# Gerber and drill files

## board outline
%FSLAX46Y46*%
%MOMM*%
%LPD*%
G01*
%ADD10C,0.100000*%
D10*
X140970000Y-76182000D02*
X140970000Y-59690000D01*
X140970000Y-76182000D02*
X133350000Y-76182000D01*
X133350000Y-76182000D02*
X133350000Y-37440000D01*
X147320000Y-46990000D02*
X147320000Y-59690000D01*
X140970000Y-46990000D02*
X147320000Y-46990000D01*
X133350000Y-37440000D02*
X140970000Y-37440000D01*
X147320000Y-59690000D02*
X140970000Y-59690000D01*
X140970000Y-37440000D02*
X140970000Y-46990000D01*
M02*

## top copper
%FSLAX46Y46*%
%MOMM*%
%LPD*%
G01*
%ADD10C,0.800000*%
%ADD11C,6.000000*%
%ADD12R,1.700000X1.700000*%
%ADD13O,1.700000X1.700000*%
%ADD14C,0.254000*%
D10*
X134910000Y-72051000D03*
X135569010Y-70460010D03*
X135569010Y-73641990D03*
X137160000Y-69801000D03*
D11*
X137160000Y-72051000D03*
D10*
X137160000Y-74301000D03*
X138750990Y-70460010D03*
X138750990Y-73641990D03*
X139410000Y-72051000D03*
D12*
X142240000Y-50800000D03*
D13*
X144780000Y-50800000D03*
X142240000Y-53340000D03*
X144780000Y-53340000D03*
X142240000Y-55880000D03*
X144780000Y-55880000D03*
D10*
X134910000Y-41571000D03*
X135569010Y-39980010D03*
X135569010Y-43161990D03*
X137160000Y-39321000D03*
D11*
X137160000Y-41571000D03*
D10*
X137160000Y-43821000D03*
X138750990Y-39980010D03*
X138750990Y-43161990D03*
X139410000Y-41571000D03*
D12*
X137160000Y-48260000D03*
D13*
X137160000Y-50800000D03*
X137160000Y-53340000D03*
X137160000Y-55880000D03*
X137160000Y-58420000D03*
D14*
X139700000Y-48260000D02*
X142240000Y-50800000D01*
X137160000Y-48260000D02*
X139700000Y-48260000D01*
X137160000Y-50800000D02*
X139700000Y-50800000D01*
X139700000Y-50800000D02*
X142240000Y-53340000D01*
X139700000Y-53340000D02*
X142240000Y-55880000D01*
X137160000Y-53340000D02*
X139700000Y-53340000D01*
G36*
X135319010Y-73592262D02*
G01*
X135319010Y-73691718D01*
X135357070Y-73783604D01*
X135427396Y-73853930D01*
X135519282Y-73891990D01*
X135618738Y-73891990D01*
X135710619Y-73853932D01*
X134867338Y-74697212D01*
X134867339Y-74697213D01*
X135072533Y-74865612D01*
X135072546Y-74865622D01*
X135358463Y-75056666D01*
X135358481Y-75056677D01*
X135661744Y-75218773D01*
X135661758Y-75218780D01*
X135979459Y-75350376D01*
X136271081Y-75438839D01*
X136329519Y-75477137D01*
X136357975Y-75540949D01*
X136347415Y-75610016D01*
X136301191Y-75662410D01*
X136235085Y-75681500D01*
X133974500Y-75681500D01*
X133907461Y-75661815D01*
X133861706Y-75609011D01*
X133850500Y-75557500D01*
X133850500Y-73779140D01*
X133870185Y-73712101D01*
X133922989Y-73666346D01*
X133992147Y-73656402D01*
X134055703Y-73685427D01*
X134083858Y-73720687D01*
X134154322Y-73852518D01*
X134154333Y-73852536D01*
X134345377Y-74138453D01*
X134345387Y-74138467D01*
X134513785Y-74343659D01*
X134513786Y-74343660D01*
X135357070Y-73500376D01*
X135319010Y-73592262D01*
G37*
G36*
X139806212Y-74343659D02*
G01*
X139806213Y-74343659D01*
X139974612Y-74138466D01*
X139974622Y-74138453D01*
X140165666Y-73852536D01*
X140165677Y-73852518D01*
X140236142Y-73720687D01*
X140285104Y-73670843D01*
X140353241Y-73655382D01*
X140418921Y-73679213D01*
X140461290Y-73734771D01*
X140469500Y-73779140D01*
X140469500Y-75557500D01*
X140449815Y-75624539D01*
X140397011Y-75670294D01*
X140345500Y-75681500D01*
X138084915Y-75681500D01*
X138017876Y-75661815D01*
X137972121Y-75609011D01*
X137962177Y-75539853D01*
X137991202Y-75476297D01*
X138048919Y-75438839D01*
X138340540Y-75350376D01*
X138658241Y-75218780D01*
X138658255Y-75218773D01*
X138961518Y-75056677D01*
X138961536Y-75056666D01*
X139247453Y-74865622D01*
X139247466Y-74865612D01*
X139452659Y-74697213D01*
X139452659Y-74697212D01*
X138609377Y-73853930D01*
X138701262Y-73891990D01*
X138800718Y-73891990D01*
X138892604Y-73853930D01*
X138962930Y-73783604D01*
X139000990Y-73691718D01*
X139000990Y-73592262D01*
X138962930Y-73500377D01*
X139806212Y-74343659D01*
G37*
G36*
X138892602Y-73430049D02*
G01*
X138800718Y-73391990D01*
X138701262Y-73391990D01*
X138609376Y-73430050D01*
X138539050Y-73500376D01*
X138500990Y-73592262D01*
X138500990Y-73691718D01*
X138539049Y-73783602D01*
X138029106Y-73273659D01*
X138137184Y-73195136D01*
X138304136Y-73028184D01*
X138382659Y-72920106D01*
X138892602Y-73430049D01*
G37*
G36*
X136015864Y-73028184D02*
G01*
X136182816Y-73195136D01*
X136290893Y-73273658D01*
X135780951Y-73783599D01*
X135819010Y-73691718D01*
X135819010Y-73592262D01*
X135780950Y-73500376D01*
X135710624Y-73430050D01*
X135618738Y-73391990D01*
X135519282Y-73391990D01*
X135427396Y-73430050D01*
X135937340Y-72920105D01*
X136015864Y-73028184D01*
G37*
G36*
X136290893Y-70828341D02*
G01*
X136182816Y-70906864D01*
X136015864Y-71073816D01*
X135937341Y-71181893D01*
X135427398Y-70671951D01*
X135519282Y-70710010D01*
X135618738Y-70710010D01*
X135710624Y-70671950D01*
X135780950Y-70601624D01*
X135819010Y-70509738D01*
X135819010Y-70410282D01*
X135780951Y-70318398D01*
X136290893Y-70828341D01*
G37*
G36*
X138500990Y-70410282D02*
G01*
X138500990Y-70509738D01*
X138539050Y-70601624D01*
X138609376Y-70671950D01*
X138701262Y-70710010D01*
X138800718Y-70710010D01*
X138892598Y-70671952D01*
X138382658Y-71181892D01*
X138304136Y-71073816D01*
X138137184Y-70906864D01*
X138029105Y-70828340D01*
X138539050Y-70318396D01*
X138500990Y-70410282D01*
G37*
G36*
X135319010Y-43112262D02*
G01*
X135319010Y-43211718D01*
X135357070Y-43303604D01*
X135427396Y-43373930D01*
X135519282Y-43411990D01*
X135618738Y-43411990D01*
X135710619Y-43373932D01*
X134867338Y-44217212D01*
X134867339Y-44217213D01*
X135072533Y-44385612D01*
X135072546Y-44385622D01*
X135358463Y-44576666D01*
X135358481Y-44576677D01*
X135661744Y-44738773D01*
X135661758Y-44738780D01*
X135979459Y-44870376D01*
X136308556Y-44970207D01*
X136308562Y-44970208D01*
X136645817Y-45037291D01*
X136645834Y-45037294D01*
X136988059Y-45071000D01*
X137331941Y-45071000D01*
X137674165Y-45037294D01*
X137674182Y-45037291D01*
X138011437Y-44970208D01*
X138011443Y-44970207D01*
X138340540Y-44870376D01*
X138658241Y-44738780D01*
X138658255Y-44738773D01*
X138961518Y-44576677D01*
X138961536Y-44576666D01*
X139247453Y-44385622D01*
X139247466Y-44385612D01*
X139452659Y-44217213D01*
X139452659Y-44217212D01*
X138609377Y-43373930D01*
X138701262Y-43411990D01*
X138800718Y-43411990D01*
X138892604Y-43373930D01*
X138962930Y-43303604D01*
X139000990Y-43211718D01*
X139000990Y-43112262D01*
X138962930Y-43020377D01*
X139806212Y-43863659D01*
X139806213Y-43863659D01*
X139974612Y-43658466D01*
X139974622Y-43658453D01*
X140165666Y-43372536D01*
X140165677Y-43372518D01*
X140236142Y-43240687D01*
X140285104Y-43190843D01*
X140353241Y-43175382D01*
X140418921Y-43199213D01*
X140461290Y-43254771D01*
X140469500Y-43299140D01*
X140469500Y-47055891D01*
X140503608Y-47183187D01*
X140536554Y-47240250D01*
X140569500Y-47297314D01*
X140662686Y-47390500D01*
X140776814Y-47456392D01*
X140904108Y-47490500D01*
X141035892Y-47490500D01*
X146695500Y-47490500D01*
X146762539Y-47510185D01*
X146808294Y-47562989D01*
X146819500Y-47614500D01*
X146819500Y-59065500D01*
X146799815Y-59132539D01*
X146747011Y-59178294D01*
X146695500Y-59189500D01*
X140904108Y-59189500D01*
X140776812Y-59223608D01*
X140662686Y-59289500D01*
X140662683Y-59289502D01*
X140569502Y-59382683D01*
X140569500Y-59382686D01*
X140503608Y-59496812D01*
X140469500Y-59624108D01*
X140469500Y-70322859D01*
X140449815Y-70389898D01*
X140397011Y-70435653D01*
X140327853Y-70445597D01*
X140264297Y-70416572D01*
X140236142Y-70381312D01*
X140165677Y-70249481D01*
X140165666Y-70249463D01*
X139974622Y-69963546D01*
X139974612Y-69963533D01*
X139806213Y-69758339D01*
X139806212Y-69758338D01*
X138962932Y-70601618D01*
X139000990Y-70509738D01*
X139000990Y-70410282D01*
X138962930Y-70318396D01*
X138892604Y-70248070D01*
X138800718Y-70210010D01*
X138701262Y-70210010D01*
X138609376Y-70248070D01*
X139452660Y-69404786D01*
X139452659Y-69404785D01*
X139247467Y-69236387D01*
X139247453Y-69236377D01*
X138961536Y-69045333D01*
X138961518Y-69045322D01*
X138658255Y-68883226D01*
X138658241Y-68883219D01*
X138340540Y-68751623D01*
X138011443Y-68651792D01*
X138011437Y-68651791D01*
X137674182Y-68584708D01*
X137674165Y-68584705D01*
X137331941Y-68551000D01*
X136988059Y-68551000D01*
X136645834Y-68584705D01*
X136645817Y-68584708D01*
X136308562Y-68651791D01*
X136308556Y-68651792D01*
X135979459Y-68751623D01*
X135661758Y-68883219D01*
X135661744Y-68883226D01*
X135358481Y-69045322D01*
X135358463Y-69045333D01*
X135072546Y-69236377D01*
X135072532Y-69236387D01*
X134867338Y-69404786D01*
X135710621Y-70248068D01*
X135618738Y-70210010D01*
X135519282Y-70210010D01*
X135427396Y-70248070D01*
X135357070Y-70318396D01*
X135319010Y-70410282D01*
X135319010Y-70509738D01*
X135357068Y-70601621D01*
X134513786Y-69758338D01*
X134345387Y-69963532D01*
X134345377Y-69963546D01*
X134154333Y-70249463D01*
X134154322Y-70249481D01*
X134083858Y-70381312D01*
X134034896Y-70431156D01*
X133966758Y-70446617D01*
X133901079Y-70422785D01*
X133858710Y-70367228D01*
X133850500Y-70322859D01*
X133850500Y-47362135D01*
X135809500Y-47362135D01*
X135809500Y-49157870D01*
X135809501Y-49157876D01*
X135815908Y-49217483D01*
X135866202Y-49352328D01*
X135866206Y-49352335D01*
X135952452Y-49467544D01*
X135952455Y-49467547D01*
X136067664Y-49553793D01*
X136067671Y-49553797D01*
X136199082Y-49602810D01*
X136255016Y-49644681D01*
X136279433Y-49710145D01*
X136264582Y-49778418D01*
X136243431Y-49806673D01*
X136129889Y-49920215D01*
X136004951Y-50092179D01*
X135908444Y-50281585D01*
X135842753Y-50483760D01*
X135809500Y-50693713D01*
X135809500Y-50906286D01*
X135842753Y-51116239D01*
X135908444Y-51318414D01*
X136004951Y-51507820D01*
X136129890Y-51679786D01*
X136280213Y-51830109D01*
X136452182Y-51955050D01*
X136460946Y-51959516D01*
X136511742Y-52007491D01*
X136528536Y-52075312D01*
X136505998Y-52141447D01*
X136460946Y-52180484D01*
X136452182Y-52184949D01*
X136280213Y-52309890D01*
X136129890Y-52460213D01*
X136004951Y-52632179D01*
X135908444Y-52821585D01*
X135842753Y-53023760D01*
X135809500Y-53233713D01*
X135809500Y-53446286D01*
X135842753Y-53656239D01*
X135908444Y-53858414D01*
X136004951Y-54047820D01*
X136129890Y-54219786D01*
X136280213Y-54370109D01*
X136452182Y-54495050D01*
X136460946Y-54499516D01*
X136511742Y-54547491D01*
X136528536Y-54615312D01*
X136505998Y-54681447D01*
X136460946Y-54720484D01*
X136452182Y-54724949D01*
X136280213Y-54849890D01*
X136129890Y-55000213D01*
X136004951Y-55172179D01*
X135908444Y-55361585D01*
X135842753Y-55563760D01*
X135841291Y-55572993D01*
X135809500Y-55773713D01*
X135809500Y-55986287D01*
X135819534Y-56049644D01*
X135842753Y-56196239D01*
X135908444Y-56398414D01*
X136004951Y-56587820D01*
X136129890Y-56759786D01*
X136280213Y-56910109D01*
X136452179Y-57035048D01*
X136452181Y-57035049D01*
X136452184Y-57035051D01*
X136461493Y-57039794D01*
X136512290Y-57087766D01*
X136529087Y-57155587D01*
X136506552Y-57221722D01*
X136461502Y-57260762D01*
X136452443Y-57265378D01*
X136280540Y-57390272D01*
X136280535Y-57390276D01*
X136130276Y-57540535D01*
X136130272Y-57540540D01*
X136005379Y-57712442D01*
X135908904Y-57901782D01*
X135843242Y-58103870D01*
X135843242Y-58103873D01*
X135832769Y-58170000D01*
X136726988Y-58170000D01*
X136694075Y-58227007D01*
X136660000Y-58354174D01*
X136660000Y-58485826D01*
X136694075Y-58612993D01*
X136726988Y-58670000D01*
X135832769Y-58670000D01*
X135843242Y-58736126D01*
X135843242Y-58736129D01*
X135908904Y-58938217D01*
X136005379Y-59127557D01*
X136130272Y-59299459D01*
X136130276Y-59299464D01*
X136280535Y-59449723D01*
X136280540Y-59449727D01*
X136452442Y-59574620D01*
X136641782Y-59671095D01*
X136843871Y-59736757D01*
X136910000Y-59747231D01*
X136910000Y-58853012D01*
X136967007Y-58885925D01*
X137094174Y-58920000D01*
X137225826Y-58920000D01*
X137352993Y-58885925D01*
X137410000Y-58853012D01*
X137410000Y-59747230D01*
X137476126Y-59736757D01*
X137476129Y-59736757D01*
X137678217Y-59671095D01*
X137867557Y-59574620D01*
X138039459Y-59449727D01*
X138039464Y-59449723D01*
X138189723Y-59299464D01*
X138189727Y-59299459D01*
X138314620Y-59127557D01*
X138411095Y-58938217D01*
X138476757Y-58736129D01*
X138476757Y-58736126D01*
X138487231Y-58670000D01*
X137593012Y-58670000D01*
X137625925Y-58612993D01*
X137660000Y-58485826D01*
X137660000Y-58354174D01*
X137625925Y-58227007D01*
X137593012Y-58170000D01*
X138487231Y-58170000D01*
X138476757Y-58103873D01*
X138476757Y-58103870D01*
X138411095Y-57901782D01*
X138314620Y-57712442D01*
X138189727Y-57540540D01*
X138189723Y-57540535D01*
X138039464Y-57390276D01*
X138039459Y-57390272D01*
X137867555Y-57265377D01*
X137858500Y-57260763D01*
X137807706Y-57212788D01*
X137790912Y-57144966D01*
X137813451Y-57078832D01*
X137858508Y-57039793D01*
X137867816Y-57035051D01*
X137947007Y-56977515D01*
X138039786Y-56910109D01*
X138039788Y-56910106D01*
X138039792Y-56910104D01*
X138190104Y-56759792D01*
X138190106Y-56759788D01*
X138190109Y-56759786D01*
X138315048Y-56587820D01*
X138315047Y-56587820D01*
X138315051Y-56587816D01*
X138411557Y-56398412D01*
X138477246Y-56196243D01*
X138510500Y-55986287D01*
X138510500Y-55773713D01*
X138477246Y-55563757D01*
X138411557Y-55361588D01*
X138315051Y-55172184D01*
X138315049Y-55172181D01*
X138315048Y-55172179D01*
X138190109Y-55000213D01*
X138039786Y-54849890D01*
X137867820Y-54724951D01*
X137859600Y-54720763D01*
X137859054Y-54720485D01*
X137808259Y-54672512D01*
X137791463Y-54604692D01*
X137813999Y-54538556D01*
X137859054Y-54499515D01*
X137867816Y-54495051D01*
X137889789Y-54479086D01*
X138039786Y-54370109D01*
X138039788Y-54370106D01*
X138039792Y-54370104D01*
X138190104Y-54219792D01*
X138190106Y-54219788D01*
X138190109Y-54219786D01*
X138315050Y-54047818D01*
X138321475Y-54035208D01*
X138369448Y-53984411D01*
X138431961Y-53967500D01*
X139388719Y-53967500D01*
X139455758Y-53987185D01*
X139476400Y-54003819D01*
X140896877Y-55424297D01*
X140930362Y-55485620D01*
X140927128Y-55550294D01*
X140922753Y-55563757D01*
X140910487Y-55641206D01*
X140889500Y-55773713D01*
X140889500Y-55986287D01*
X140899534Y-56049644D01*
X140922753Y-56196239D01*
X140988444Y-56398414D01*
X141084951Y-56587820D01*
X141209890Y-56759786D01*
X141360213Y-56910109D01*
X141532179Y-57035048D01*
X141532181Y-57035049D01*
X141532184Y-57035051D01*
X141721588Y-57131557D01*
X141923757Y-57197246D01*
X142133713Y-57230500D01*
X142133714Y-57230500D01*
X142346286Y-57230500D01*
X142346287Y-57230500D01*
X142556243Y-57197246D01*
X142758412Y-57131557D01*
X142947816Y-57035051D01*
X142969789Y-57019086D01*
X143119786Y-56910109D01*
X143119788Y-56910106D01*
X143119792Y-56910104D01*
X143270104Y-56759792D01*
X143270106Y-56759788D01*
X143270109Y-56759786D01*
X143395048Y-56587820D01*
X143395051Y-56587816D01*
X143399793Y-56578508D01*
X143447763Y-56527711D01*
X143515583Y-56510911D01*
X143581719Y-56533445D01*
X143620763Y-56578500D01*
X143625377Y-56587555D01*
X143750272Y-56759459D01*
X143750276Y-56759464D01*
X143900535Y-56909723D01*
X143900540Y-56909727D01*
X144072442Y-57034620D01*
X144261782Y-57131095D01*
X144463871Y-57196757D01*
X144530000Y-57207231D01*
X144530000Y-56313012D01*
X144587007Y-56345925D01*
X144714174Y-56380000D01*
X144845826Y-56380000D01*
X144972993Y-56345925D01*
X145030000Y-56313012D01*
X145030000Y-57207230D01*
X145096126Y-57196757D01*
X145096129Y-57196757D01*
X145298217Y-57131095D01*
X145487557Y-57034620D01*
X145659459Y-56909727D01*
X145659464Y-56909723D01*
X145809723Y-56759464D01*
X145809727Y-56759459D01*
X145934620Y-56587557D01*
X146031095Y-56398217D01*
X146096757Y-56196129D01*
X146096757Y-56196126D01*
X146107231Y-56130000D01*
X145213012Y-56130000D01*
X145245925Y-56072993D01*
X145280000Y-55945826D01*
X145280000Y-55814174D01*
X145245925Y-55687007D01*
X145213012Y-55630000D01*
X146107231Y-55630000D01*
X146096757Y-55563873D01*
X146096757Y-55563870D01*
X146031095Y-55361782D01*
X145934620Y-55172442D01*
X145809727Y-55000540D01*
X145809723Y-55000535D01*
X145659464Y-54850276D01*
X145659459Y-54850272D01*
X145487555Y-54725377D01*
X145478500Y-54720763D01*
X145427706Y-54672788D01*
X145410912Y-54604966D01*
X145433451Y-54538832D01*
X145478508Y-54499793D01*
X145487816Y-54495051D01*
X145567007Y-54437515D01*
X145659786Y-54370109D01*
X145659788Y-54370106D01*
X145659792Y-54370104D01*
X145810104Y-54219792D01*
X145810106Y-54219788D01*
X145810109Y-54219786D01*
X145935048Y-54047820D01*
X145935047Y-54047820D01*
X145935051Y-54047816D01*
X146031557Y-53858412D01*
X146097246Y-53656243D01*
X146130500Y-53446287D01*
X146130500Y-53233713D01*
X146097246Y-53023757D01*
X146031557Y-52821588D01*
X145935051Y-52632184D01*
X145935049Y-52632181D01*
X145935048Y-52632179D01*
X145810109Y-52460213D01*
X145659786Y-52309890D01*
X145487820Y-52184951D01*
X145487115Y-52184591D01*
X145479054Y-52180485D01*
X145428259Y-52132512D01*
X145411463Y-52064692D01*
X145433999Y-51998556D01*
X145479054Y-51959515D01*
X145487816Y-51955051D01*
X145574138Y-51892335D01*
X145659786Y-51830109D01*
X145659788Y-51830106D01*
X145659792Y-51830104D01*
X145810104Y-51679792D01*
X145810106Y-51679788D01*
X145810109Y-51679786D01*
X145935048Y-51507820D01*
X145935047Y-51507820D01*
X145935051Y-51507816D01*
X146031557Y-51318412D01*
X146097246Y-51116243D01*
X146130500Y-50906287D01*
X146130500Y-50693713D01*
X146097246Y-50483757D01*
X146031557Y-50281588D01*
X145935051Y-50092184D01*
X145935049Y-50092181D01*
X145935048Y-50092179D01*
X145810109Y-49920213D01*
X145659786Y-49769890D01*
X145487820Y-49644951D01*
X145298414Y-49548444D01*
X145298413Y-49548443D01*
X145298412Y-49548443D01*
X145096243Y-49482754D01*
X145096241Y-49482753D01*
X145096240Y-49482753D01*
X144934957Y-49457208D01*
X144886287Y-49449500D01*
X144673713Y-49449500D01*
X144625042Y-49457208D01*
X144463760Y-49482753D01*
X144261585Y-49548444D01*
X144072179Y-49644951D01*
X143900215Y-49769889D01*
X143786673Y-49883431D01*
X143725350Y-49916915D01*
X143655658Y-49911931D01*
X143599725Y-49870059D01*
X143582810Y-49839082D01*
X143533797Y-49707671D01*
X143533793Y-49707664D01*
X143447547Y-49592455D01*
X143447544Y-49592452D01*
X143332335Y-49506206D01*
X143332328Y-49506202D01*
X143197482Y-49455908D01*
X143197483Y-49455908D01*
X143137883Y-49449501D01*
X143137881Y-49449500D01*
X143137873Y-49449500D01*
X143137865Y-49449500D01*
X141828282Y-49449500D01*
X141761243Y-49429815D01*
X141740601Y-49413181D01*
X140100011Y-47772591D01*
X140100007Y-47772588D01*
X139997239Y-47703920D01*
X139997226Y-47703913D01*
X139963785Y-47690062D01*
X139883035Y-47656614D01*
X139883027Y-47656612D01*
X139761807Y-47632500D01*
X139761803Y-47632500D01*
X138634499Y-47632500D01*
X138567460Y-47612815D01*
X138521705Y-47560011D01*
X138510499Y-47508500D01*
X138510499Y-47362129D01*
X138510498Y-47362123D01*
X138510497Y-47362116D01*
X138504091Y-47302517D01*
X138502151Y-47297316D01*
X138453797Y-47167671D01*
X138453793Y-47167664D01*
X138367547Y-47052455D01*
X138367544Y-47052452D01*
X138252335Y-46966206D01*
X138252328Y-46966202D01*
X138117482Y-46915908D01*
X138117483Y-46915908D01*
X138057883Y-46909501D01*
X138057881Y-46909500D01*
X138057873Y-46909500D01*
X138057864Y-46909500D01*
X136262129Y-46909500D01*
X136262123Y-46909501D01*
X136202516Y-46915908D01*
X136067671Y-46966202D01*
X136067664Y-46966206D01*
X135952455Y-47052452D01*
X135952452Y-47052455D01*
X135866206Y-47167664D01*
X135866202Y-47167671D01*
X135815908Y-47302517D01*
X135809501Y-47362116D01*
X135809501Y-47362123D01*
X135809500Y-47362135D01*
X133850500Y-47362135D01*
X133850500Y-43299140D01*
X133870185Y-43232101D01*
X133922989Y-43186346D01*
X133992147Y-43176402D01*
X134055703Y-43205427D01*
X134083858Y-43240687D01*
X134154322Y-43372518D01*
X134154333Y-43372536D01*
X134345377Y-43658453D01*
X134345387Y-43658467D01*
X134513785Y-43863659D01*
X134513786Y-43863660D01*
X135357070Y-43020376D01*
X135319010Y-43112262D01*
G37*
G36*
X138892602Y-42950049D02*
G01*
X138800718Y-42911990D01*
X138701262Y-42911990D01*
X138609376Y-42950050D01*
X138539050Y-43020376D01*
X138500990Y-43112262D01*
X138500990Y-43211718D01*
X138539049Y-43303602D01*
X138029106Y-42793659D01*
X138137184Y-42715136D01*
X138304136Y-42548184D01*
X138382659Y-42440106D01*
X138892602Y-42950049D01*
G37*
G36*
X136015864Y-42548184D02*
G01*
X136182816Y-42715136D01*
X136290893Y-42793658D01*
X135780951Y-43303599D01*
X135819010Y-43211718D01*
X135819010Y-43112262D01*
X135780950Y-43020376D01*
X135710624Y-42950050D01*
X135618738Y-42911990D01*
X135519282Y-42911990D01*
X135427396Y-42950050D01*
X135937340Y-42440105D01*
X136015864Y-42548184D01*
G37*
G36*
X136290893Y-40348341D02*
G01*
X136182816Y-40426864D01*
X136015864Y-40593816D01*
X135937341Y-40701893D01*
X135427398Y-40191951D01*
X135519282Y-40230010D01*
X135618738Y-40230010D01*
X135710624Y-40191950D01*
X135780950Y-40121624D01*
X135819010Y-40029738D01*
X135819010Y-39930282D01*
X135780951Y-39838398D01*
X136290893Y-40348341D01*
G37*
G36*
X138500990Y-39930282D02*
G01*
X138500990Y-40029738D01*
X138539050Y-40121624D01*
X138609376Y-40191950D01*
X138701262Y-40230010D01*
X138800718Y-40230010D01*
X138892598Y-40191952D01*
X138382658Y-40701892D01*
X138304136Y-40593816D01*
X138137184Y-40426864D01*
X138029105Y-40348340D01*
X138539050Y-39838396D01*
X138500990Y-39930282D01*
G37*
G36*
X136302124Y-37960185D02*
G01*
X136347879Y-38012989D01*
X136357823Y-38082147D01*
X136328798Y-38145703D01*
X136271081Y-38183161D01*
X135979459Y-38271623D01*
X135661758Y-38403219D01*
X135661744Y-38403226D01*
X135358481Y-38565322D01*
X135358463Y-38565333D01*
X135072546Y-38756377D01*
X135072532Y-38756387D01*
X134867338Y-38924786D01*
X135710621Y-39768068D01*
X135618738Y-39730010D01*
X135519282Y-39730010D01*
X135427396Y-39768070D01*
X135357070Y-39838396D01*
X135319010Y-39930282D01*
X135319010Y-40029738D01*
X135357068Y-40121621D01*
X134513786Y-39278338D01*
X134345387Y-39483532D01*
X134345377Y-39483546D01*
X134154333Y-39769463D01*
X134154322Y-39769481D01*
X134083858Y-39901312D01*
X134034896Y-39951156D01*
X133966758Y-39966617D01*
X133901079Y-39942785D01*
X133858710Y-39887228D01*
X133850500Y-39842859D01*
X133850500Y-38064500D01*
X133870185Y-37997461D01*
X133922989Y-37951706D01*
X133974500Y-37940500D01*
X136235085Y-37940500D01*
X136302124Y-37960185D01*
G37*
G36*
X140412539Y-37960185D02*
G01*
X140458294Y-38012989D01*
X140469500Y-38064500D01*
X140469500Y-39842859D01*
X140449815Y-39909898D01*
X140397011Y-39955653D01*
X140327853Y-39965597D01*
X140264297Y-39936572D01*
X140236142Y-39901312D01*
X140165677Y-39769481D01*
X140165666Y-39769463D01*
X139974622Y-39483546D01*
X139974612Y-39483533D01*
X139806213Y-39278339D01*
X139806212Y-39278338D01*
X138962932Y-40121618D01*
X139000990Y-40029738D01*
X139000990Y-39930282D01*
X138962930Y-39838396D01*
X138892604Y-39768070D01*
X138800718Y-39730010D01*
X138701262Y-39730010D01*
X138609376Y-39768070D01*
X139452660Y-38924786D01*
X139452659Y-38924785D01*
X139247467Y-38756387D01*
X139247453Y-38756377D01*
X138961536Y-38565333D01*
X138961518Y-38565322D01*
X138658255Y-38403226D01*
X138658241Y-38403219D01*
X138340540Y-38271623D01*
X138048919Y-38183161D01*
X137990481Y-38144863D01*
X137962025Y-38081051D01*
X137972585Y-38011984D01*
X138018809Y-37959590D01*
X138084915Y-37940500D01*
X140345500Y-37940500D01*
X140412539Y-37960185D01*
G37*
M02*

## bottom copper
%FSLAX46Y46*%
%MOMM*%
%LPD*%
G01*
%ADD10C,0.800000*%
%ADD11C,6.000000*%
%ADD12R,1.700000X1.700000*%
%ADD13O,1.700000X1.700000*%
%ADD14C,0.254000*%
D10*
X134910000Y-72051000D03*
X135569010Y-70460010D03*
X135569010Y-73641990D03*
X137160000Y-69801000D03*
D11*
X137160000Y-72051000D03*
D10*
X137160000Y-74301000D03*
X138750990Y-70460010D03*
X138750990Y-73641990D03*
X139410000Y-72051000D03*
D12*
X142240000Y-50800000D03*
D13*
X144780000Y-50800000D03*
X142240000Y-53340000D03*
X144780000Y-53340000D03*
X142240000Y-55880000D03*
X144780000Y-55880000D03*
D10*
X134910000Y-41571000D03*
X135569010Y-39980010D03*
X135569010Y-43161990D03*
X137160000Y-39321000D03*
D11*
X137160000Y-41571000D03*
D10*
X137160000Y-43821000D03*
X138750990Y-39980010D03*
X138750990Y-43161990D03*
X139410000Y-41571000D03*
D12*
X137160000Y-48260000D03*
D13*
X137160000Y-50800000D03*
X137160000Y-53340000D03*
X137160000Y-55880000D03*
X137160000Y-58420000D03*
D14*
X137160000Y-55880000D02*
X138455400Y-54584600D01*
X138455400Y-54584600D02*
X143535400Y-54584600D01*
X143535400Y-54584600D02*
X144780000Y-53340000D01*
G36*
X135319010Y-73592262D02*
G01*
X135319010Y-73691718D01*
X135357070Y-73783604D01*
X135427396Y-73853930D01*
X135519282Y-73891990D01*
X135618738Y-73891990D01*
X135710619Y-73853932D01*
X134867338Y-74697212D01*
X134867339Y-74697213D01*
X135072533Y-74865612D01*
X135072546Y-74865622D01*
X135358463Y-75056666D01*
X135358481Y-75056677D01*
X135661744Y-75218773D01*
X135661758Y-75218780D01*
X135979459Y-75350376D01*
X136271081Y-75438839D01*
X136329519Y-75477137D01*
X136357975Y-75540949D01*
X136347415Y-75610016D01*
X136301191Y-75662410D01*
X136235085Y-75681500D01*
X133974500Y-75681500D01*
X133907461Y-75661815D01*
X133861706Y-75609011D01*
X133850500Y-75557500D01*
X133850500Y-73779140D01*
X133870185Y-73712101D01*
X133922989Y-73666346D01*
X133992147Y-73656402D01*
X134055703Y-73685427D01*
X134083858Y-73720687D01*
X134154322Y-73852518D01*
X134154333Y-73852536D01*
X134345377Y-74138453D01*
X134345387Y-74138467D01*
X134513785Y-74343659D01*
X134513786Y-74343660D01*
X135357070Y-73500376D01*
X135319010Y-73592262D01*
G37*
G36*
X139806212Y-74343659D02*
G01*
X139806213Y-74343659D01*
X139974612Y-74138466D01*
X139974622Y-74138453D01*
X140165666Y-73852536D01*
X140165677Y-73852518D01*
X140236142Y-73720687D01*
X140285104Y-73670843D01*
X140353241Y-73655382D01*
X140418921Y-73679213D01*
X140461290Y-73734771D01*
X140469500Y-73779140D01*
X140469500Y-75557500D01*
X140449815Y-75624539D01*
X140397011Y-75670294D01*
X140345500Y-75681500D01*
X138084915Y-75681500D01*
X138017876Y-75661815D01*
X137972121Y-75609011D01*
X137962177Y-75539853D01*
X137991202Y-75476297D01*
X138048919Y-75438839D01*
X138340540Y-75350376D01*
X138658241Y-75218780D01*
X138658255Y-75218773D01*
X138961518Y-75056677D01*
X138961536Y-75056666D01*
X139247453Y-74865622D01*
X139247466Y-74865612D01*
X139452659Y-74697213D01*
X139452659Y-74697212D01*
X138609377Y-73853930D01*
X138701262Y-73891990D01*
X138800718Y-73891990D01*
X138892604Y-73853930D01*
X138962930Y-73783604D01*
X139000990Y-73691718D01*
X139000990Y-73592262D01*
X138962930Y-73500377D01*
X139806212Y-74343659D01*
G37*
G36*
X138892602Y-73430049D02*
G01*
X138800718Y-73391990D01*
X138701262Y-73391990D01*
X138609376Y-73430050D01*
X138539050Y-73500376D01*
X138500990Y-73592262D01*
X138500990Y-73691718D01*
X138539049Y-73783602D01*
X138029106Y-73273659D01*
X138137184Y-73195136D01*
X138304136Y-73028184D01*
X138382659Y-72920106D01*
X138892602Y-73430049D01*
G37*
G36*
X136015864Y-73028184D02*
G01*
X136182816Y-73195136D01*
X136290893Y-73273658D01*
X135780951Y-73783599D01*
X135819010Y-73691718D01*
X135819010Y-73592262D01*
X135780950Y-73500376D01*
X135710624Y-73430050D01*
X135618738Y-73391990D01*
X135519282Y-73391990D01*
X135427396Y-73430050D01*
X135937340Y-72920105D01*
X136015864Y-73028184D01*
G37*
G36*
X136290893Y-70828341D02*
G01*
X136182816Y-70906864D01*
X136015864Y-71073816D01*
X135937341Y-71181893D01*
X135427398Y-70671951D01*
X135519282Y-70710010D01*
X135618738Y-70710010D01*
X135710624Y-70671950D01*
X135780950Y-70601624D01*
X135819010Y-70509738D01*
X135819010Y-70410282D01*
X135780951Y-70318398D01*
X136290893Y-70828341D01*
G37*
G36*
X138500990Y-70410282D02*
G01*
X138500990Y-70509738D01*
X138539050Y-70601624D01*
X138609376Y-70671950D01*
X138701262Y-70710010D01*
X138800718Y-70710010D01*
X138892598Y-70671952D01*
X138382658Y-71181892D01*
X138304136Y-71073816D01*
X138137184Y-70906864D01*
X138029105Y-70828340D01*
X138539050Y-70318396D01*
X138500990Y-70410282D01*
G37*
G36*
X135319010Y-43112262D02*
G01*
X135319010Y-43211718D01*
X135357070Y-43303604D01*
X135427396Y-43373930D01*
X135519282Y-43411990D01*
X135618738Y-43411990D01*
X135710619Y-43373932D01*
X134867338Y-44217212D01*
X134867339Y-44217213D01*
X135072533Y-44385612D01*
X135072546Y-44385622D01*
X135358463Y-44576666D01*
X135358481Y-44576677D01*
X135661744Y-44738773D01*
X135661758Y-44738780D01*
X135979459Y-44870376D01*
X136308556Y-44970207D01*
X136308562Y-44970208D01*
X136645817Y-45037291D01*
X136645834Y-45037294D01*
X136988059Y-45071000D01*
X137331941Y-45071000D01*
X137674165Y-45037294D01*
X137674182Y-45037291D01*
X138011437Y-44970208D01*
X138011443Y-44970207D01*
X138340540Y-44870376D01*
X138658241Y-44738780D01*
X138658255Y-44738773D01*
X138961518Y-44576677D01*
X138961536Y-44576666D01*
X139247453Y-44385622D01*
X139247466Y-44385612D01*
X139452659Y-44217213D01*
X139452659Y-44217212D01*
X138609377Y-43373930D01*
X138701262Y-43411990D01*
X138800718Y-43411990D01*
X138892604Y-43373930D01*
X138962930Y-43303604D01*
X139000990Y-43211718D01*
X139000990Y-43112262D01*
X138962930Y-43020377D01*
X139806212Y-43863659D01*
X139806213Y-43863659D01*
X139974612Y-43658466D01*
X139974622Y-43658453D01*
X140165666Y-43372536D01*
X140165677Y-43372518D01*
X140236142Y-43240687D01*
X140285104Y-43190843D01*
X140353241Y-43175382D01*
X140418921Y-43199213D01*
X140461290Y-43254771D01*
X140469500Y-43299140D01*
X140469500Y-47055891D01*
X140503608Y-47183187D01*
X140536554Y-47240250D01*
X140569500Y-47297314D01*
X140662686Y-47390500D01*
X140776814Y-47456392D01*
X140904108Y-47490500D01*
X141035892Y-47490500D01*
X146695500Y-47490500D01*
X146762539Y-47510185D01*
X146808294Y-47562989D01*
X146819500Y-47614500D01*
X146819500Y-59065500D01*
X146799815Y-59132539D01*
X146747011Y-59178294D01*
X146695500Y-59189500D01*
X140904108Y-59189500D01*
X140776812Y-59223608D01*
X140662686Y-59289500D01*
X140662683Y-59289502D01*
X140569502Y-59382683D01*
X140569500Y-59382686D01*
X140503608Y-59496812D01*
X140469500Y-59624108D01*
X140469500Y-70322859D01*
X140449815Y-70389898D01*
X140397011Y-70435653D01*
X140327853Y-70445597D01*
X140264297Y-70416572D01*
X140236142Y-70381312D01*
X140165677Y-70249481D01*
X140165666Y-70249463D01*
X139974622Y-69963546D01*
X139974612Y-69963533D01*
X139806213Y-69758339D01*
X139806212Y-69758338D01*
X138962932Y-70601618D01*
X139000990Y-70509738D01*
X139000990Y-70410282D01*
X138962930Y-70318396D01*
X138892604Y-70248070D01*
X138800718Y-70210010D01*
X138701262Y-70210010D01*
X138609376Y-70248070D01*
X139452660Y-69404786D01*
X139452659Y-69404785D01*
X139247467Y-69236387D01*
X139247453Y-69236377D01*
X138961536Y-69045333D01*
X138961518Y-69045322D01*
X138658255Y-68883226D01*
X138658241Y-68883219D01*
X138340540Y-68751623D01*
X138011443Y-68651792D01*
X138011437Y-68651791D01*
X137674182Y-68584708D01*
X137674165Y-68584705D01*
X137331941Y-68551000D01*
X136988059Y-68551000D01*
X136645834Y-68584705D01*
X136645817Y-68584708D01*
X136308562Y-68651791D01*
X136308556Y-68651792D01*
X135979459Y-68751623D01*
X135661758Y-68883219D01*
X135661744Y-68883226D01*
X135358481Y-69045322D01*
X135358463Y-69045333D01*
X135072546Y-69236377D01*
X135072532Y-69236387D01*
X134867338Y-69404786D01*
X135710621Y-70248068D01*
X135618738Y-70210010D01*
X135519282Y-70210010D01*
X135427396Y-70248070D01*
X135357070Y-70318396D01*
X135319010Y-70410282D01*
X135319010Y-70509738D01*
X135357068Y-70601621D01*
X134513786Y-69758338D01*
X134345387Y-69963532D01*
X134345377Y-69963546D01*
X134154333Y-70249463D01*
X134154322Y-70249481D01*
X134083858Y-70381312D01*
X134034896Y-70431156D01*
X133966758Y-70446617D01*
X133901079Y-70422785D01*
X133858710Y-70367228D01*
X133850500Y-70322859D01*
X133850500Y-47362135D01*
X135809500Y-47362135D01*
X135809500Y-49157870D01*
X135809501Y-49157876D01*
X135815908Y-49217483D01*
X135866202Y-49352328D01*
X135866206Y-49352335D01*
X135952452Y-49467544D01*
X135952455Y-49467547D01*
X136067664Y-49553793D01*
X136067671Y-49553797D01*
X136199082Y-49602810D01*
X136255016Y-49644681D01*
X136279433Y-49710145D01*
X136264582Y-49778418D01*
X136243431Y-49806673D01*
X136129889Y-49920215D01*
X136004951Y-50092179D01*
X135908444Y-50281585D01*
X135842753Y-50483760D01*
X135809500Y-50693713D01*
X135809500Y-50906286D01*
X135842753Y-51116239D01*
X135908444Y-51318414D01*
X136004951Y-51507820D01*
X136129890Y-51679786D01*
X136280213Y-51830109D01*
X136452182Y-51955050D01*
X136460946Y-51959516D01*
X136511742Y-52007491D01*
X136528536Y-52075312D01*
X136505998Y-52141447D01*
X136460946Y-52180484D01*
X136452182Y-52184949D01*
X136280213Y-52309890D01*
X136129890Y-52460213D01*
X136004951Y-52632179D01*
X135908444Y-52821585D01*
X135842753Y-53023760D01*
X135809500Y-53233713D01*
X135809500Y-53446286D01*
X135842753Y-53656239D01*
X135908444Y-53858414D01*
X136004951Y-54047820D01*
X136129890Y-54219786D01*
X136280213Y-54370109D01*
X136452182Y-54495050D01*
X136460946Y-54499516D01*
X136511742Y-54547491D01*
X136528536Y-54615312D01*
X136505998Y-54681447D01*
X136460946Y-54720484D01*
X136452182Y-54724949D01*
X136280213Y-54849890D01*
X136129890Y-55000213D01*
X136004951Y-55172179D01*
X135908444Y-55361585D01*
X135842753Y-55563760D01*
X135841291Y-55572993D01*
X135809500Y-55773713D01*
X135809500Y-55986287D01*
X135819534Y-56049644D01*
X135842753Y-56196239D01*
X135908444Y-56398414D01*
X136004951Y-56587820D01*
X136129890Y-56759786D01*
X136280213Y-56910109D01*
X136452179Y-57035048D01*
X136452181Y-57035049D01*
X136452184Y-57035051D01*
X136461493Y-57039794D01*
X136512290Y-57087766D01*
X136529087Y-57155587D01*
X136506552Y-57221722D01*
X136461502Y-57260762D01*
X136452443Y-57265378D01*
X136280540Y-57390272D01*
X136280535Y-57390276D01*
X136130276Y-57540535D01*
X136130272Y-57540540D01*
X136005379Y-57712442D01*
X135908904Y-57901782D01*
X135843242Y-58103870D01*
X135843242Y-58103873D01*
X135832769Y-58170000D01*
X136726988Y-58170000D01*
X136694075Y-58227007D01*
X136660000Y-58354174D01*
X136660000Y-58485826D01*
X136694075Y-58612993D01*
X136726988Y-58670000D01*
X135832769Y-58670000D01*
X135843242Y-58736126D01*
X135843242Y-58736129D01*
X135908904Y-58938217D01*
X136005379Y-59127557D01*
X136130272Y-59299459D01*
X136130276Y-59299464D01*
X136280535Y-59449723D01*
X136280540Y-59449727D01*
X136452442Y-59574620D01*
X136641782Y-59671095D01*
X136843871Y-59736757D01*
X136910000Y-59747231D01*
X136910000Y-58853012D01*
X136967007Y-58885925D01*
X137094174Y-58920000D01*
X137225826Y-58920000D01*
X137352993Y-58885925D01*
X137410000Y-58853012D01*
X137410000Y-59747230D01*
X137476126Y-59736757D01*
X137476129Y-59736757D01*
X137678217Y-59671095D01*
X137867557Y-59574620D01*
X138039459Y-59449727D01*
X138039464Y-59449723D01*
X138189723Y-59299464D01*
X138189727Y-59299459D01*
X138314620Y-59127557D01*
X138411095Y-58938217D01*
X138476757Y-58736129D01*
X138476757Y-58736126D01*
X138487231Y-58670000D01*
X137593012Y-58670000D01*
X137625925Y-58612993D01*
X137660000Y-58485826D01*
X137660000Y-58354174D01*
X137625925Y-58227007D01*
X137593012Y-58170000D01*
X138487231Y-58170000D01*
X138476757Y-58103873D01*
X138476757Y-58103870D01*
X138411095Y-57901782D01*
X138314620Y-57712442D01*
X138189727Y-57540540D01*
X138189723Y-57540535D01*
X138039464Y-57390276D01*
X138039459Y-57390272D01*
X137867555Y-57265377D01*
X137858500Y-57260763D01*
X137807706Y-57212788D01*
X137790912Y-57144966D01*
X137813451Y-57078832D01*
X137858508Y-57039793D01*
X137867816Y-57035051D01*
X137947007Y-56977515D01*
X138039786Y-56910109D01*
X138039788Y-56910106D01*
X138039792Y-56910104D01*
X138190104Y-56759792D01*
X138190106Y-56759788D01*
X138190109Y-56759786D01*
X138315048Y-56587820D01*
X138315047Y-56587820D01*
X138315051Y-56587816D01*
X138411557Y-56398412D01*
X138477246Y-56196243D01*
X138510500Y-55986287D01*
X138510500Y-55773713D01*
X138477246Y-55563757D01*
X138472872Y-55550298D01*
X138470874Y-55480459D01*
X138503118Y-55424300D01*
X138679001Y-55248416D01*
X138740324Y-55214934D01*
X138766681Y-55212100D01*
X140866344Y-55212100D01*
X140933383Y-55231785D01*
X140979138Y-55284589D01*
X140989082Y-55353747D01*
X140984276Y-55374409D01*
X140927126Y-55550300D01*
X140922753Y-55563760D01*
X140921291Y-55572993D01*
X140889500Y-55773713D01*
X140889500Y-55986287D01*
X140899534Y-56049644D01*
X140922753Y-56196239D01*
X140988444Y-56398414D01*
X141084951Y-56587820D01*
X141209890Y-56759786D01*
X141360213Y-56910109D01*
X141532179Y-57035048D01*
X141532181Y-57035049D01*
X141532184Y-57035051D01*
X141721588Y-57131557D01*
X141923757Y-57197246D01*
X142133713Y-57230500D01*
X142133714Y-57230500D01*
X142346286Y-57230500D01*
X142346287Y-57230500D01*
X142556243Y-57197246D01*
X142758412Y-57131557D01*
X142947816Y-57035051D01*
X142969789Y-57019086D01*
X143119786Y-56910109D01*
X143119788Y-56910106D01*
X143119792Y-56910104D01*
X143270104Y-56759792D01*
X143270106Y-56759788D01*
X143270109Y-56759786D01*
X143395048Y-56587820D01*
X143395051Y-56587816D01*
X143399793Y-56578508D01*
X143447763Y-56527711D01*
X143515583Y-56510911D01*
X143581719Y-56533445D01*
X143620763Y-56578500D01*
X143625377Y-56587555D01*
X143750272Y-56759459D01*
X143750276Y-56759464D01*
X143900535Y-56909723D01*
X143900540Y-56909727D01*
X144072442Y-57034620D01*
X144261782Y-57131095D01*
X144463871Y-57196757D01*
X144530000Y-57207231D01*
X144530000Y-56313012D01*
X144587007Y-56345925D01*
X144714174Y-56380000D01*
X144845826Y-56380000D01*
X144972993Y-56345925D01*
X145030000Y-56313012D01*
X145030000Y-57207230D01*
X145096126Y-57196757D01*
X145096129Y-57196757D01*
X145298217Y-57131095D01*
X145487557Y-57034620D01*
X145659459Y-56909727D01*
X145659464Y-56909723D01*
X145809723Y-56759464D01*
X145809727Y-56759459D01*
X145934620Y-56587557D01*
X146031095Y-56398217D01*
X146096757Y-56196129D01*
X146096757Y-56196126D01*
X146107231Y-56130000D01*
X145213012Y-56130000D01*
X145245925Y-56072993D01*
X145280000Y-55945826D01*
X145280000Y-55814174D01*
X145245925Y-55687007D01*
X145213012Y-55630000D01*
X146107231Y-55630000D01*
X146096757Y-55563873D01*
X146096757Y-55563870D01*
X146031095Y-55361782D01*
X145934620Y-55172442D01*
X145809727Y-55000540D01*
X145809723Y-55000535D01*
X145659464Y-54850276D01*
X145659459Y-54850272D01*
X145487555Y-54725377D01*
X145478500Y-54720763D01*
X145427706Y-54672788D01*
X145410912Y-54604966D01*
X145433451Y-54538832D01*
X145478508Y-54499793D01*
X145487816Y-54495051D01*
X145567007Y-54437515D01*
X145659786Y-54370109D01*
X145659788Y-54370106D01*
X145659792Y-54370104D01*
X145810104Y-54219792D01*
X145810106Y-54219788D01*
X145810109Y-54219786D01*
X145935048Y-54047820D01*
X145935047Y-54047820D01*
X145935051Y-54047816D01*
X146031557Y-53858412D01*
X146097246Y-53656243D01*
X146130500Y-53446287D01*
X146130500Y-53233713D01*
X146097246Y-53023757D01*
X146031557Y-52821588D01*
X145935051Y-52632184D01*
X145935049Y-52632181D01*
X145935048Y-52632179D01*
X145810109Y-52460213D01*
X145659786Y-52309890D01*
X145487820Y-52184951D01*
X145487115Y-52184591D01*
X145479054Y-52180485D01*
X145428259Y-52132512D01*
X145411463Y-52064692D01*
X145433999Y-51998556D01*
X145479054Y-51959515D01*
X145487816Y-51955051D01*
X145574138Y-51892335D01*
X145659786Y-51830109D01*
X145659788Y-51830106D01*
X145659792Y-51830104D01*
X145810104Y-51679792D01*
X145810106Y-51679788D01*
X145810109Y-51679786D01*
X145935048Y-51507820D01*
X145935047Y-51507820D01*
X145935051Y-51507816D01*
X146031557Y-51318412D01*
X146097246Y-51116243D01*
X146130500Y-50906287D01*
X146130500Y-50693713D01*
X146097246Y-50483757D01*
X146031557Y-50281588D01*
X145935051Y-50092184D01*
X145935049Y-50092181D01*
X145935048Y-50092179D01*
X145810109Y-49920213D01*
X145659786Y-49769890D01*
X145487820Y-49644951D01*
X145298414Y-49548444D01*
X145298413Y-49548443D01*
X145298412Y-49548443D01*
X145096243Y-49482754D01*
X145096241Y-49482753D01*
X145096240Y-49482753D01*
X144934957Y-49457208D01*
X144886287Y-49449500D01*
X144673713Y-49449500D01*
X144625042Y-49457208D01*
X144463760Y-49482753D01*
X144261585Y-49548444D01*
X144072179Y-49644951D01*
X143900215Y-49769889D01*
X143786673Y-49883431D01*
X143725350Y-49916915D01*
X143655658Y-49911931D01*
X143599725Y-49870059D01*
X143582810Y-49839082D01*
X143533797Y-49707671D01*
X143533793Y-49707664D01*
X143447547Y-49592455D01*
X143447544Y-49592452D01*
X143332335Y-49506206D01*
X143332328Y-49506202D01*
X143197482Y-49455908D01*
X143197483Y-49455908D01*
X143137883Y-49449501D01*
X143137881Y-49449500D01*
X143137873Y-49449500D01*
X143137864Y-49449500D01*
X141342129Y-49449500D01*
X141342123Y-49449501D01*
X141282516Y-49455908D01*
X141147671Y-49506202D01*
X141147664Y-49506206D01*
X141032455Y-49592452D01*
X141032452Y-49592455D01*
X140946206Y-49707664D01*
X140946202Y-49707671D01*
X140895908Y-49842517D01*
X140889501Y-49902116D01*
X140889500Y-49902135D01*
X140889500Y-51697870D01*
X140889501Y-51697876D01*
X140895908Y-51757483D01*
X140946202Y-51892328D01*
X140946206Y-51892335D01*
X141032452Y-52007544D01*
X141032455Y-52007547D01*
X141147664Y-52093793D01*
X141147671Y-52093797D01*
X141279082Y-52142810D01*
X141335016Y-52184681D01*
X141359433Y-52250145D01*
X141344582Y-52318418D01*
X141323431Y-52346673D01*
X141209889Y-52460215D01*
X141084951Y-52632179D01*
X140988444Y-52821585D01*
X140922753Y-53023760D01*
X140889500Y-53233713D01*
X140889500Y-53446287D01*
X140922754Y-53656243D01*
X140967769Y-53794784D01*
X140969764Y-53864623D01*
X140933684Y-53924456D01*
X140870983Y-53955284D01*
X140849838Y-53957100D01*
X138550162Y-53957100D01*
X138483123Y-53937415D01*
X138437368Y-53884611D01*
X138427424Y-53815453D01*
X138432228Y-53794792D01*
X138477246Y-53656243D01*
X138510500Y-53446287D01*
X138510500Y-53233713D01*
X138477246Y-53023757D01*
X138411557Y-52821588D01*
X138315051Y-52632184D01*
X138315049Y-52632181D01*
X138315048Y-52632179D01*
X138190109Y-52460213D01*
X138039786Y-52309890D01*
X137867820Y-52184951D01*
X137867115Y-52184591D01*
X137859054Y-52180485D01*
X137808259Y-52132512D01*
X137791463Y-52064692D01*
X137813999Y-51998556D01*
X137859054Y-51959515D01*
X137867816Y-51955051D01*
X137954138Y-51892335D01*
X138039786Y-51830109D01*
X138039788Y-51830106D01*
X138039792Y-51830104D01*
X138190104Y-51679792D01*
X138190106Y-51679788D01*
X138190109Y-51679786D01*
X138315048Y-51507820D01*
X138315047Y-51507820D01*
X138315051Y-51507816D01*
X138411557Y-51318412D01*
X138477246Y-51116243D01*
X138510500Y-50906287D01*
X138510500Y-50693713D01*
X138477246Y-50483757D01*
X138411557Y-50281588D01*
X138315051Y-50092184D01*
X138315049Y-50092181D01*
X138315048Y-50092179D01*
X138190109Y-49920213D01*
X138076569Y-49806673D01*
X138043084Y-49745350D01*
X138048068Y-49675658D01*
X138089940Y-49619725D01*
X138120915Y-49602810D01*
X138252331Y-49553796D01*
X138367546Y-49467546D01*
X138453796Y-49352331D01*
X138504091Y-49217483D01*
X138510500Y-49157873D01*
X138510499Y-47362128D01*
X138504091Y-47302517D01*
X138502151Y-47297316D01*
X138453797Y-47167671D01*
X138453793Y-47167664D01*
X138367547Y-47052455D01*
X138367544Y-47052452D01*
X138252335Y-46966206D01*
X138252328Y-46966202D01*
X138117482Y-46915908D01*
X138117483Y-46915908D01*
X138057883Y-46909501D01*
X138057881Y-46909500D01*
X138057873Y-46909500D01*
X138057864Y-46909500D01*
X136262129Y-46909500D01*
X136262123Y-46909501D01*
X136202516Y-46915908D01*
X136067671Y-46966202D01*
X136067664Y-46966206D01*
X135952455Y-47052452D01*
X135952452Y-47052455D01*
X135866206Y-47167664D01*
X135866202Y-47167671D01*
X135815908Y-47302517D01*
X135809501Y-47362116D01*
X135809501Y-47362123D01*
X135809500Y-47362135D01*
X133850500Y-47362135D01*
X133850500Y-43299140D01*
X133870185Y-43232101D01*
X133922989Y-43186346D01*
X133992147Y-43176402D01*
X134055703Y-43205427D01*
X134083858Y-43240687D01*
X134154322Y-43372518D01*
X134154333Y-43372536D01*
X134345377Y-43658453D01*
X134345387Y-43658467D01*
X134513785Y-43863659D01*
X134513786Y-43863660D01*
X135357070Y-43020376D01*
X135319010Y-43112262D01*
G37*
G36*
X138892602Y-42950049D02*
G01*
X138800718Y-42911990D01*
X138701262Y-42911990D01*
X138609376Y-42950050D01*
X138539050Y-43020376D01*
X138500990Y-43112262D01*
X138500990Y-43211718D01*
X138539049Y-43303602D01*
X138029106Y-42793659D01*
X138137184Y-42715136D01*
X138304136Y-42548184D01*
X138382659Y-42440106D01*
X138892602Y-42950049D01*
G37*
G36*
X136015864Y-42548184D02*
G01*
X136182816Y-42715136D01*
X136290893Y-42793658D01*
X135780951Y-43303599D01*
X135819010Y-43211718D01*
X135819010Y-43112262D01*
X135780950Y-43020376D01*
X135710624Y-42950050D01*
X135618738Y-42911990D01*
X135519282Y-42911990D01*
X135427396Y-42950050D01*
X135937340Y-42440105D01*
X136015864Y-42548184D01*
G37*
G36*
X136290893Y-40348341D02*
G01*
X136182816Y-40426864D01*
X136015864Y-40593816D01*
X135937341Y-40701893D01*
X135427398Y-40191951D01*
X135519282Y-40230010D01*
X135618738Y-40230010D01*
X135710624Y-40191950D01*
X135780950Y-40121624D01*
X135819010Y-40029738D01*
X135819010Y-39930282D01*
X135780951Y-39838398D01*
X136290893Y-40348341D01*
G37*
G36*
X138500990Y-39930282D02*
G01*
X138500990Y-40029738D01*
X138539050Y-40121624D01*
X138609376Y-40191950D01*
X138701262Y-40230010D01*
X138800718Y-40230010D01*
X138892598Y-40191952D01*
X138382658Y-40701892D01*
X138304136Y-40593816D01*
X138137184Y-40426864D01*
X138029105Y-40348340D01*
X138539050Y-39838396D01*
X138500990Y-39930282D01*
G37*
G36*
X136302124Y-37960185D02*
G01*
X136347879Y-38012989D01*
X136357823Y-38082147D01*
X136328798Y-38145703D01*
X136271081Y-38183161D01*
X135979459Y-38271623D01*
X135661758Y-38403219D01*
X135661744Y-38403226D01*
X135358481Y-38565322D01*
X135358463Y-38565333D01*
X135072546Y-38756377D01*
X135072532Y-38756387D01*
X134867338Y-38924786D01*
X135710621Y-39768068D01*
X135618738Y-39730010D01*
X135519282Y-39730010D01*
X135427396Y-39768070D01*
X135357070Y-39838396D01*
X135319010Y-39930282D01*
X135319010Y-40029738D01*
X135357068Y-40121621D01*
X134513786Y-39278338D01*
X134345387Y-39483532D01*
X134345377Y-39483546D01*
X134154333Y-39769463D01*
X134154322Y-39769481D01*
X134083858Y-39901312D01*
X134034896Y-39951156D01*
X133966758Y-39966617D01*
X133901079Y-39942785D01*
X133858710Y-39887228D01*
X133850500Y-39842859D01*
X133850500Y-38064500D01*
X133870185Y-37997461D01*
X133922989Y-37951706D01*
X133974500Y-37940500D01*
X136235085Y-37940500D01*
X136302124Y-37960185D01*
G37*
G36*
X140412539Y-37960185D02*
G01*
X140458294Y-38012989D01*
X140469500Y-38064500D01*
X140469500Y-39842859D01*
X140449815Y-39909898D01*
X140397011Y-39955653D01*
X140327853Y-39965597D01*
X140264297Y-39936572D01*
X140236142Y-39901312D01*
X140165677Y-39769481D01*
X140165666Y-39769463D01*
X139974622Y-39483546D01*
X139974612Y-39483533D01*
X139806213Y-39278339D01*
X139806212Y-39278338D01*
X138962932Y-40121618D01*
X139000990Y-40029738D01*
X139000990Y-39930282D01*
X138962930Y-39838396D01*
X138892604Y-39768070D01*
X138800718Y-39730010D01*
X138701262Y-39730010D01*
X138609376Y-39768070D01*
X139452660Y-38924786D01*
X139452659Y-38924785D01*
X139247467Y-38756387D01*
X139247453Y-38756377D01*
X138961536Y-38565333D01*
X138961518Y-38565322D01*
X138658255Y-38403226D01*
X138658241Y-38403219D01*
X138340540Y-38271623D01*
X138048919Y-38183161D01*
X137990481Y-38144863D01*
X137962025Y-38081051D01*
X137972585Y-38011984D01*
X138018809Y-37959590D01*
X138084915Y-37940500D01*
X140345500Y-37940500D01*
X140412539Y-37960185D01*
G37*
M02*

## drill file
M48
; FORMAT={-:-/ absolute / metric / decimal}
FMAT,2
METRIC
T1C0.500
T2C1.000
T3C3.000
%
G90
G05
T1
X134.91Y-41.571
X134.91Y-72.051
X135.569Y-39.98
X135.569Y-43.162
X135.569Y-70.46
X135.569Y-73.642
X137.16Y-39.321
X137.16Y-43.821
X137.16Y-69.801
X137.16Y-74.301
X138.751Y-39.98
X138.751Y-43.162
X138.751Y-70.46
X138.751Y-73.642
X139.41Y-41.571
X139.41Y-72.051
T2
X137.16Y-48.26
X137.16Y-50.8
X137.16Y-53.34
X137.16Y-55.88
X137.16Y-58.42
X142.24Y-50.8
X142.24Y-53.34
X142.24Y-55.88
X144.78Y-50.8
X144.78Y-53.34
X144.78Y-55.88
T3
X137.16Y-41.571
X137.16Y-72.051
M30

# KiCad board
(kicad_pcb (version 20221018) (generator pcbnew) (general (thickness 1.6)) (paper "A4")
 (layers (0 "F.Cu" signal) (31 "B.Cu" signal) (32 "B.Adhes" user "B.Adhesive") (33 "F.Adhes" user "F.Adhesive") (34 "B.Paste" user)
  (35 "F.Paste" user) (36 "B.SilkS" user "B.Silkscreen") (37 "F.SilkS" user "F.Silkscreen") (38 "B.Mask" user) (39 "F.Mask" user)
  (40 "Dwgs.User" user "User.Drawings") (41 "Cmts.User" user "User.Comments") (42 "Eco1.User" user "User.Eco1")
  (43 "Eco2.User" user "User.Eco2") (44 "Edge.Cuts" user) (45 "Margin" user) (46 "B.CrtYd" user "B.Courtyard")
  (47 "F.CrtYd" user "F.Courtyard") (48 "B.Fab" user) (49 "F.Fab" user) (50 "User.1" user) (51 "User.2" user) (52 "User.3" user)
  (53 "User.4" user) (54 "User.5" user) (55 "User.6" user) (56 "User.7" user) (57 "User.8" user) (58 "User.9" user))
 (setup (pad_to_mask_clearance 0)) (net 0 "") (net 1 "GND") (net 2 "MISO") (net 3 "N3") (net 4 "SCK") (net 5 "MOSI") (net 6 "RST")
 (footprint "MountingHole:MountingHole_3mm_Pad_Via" (layer "F.Cu") (at 137.16 72.051)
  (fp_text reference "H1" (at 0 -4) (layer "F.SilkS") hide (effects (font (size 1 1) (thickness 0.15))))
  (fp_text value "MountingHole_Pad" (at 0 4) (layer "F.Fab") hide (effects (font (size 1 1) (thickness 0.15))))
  (pad "1" thru_hole circle (at -2.25 0) (size 0.8 0.8) (drill 0.5) (layers "*.Cu" "*.Mask") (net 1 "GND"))
  (pad "1" thru_hole circle (at -1.59099 -1.59099) (size 0.8 0.8) (drill 0.5) (layers "*.Cu" "*.Mask") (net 1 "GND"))
  (pad "1" thru_hole circle (at -1.59099 1.59099) (size 0.8 0.8) (drill 0.5) (layers "*.Cu" "*.Mask") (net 1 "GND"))
  (pad "1" thru_hole circle (at 0 -2.25) (size 0.8 0.8) (drill 0.5) (layers "*.Cu" "*.Mask") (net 1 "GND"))
  (pad "1" thru_hole circle (at 0 0) (size 6 6) (drill 3) (layers "*.Cu" "*.Mask") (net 1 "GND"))
  (pad "1" thru_hole circle (at 0 2.25) (size 0.8 0.8) (drill 0.5) (layers "*.Cu" "*.Mask") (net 1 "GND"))
  (pad "1" thru_hole circle (at 1.59099 -1.59099) (size 0.8 0.8) (drill 0.5) (layers "*.Cu" "*.Mask") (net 1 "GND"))
  (pad "1" thru_hole circle (at 1.59099 1.59099) (size 0.8 0.8) (drill 0.5) (layers "*.Cu" "*.Mask") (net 1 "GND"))
  (pad "1" thru_hole circle (at 2.25 0) (size 0.8 0.8) (drill 0.5) (layers "*.Cu" "*.Mask") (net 1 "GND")))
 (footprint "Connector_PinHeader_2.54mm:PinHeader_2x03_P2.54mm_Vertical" (layer "F.Cu") (at 142.24 50.8)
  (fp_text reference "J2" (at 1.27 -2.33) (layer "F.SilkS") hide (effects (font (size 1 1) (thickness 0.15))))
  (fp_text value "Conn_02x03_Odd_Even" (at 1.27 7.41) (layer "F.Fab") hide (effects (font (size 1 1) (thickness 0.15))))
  (pad "1" thru_hole rect (at 0 0) (size 1.7 1.7) (drill 1) (layers "*.Cu" "*.Mask") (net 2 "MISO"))
  (pad "2" thru_hole oval (at 2.54 0) (size 1.7 1.7) (drill 1) (layers "*.Cu" "*.Mask") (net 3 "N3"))
  (pad "3" thru_hole oval (at 0 2.54) (size 1.7 1.7) (drill 1) (layers "*.Cu" "*.Mask") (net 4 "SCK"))
  (pad "4" thru_hole oval (at 2.54 2.54) (size 1.7 1.7) (drill 1) (layers "*.Cu" "*.Mask") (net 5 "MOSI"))
  (pad "5" thru_hole oval (at 0 5.08) (size 1.7 1.7) (drill 1) (layers "*.Cu" "*.Mask") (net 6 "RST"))
  (pad "6" thru_hole oval (at 2.54 5.08) (size 1.7 1.7) (drill 1) (layers "*.Cu" "*.Mask") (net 1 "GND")))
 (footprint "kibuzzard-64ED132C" (layer "F.Cu") (at 137.16 64.262 -90)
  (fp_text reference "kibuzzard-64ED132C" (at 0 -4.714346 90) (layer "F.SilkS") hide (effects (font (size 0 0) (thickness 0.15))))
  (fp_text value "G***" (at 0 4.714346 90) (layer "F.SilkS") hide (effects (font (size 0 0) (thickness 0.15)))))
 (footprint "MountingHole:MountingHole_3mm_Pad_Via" (layer "F.Cu") (at 137.16 41.571)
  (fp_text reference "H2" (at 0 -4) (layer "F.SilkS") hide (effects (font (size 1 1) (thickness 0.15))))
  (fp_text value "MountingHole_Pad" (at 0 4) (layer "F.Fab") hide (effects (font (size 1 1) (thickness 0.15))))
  (pad "1" thru_hole circle (at -2.25 0) (size 0.8 0.8) (drill 0.5) (layers "*.Cu" "*.Mask") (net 1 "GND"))
  (pad "1" thru_hole circle (at -1.59099 -1.59099) (size 0.8 0.8) (drill 0.5) (layers "*.Cu" "*.Mask") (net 1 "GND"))
  (pad "1" thru_hole circle (at -1.59099 1.59099) (size 0.8 0.8) (drill 0.5) (layers "*.Cu" "*.Mask") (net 1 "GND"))
  (pad "1" thru_hole circle (at 0 -2.25) (size 0.8 0.8) (drill 0.5) (layers "*.Cu" "*.Mask") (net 1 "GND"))
  (pad "1" thru_hole circle (at 0 0) (size 6 6) (drill 3) (layers "*.Cu" "*.Mask") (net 1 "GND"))
  (pad "1" thru_hole circle (at 0 2.25) (size 0.8 0.8) (drill 0.5) (layers "*.Cu" "*.Mask") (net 1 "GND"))
  (pad "1" thru_hole circle (at 1.59099 -1.59099) (size 0.8 0.8) (drill 0.5) (layers "*.Cu" "*.Mask") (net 1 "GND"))
  (pad "1" thru_hole circle (at 1.59099 1.59099) (size 0.8 0.8) (drill 0.5) (layers "*.Cu" "*.Mask") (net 1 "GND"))
  (pad "1" thru_hole circle (at 2.25 0) (size 0.8 0.8) (drill 0.5) (layers "*.Cu" "*.Mask") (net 1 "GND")))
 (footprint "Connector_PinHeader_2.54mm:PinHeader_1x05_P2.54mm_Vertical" (layer "B.Cu") (at 137.16 48.26 180)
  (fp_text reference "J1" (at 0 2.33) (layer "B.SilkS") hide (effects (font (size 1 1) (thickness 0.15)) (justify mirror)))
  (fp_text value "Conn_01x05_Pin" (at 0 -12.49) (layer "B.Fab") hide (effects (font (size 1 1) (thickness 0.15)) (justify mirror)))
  (pad "1" thru_hole rect (at 0 0 180) (size 1.7 1.7) (drill 1) (layers "*.Cu" "*.Mask") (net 2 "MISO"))
  (pad "2" thru_hole oval (at 0 -2.54 180) (size 1.7 1.7) (drill 1) (layers "*.Cu" "*.Mask") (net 4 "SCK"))
  (pad "3" thru_hole oval (at 0 -5.08 180) (size 1.7 1.7) (drill 1) (layers "*.Cu" "*.Mask") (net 6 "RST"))
  (pad "4" thru_hole oval (at 0 -7.62 180) (size 1.7 1.7) (drill 1) (layers "*.Cu" "*.Mask") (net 5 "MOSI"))
  (pad "5" thru_hole oval (at 0 -10.16 180) (size 1.7 1.7) (drill 1) (layers "*.Cu" "*.Mask") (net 1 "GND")))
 (gr_line (start 140.97 76.182) (end 140.97 59.69) (stroke (width 0.1) (type default)) (layer "Edge.Cuts"))
 (gr_line (start 140.97 76.182) (end 133.35 76.182) (stroke (width 0.1) (type default)) (layer "Edge.Cuts"))
 (gr_line (start 133.35 76.182) (end 133.35 37.44) (stroke (width 0.1) (type default)) (layer "Edge.Cuts"))
 (gr_line (start 147.32 46.99) (end 147.32 59.69) (stroke (width 0.1) (type default)) (layer "Edge.Cuts"))
 (gr_line (start 140.97 46.99) (end 147.32 46.99) (stroke (width 0.1) (type default)) (layer "Edge.Cuts"))
 (gr_line (start 133.35 37.44) (end 140.97 37.44) (stroke (width 0.1) (type default)) (layer "Edge.Cuts"))
 (gr_line (start 147.32 59.69) (end 140.97 59.69) (stroke (width 0.1) (type default)) (layer "Edge.Cuts"))
 (gr_line (start 140.97 37.44) (end 140.97 46.99) (stroke (width 0.1) (type default)) (layer "Edge.Cuts"))
 (segment (start 139.7 48.26) (end 142.24 50.8) (width 0.254) (layer "F.Cu") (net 2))
 (segment (start 137.16 48.26) (end 139.7 48.26) (width 0.254) (layer "F.Cu") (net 2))
 (segment (start 137.16 50.8) (end 139.7 50.8) (width 0.254) (layer "F.Cu") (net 4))
 (segment (start 139.7 50.8) (end 142.24 53.34) (width 0.254) (layer "F.Cu") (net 4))
 (segment (start 139.7 53.34) (end 142.24 55.88) (width 0.254) (layer "F.Cu") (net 6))
 (segment (start 137.16 53.34) (end 139.7 53.34) (width 0.254) (layer "F.Cu") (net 6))
 (segment (start 137.16 55.88) (end 138.4554 54.5846) (width 0.254) (layer "B.Cu") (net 5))
 (segment (start 138.4554 54.5846) (end 143.5354 54.5846) (width 0.254) (layer "B.Cu") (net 5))
 (segment (start 143.5354 54.5846) (end 144.78 53.34) (width 0.254) (layer "B.Cu") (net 5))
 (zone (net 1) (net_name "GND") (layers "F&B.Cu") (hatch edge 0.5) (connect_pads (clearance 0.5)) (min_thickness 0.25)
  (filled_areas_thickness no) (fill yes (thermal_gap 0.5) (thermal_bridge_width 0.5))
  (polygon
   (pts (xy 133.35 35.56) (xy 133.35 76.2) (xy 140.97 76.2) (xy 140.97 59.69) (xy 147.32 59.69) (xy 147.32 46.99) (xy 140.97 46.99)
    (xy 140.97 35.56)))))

